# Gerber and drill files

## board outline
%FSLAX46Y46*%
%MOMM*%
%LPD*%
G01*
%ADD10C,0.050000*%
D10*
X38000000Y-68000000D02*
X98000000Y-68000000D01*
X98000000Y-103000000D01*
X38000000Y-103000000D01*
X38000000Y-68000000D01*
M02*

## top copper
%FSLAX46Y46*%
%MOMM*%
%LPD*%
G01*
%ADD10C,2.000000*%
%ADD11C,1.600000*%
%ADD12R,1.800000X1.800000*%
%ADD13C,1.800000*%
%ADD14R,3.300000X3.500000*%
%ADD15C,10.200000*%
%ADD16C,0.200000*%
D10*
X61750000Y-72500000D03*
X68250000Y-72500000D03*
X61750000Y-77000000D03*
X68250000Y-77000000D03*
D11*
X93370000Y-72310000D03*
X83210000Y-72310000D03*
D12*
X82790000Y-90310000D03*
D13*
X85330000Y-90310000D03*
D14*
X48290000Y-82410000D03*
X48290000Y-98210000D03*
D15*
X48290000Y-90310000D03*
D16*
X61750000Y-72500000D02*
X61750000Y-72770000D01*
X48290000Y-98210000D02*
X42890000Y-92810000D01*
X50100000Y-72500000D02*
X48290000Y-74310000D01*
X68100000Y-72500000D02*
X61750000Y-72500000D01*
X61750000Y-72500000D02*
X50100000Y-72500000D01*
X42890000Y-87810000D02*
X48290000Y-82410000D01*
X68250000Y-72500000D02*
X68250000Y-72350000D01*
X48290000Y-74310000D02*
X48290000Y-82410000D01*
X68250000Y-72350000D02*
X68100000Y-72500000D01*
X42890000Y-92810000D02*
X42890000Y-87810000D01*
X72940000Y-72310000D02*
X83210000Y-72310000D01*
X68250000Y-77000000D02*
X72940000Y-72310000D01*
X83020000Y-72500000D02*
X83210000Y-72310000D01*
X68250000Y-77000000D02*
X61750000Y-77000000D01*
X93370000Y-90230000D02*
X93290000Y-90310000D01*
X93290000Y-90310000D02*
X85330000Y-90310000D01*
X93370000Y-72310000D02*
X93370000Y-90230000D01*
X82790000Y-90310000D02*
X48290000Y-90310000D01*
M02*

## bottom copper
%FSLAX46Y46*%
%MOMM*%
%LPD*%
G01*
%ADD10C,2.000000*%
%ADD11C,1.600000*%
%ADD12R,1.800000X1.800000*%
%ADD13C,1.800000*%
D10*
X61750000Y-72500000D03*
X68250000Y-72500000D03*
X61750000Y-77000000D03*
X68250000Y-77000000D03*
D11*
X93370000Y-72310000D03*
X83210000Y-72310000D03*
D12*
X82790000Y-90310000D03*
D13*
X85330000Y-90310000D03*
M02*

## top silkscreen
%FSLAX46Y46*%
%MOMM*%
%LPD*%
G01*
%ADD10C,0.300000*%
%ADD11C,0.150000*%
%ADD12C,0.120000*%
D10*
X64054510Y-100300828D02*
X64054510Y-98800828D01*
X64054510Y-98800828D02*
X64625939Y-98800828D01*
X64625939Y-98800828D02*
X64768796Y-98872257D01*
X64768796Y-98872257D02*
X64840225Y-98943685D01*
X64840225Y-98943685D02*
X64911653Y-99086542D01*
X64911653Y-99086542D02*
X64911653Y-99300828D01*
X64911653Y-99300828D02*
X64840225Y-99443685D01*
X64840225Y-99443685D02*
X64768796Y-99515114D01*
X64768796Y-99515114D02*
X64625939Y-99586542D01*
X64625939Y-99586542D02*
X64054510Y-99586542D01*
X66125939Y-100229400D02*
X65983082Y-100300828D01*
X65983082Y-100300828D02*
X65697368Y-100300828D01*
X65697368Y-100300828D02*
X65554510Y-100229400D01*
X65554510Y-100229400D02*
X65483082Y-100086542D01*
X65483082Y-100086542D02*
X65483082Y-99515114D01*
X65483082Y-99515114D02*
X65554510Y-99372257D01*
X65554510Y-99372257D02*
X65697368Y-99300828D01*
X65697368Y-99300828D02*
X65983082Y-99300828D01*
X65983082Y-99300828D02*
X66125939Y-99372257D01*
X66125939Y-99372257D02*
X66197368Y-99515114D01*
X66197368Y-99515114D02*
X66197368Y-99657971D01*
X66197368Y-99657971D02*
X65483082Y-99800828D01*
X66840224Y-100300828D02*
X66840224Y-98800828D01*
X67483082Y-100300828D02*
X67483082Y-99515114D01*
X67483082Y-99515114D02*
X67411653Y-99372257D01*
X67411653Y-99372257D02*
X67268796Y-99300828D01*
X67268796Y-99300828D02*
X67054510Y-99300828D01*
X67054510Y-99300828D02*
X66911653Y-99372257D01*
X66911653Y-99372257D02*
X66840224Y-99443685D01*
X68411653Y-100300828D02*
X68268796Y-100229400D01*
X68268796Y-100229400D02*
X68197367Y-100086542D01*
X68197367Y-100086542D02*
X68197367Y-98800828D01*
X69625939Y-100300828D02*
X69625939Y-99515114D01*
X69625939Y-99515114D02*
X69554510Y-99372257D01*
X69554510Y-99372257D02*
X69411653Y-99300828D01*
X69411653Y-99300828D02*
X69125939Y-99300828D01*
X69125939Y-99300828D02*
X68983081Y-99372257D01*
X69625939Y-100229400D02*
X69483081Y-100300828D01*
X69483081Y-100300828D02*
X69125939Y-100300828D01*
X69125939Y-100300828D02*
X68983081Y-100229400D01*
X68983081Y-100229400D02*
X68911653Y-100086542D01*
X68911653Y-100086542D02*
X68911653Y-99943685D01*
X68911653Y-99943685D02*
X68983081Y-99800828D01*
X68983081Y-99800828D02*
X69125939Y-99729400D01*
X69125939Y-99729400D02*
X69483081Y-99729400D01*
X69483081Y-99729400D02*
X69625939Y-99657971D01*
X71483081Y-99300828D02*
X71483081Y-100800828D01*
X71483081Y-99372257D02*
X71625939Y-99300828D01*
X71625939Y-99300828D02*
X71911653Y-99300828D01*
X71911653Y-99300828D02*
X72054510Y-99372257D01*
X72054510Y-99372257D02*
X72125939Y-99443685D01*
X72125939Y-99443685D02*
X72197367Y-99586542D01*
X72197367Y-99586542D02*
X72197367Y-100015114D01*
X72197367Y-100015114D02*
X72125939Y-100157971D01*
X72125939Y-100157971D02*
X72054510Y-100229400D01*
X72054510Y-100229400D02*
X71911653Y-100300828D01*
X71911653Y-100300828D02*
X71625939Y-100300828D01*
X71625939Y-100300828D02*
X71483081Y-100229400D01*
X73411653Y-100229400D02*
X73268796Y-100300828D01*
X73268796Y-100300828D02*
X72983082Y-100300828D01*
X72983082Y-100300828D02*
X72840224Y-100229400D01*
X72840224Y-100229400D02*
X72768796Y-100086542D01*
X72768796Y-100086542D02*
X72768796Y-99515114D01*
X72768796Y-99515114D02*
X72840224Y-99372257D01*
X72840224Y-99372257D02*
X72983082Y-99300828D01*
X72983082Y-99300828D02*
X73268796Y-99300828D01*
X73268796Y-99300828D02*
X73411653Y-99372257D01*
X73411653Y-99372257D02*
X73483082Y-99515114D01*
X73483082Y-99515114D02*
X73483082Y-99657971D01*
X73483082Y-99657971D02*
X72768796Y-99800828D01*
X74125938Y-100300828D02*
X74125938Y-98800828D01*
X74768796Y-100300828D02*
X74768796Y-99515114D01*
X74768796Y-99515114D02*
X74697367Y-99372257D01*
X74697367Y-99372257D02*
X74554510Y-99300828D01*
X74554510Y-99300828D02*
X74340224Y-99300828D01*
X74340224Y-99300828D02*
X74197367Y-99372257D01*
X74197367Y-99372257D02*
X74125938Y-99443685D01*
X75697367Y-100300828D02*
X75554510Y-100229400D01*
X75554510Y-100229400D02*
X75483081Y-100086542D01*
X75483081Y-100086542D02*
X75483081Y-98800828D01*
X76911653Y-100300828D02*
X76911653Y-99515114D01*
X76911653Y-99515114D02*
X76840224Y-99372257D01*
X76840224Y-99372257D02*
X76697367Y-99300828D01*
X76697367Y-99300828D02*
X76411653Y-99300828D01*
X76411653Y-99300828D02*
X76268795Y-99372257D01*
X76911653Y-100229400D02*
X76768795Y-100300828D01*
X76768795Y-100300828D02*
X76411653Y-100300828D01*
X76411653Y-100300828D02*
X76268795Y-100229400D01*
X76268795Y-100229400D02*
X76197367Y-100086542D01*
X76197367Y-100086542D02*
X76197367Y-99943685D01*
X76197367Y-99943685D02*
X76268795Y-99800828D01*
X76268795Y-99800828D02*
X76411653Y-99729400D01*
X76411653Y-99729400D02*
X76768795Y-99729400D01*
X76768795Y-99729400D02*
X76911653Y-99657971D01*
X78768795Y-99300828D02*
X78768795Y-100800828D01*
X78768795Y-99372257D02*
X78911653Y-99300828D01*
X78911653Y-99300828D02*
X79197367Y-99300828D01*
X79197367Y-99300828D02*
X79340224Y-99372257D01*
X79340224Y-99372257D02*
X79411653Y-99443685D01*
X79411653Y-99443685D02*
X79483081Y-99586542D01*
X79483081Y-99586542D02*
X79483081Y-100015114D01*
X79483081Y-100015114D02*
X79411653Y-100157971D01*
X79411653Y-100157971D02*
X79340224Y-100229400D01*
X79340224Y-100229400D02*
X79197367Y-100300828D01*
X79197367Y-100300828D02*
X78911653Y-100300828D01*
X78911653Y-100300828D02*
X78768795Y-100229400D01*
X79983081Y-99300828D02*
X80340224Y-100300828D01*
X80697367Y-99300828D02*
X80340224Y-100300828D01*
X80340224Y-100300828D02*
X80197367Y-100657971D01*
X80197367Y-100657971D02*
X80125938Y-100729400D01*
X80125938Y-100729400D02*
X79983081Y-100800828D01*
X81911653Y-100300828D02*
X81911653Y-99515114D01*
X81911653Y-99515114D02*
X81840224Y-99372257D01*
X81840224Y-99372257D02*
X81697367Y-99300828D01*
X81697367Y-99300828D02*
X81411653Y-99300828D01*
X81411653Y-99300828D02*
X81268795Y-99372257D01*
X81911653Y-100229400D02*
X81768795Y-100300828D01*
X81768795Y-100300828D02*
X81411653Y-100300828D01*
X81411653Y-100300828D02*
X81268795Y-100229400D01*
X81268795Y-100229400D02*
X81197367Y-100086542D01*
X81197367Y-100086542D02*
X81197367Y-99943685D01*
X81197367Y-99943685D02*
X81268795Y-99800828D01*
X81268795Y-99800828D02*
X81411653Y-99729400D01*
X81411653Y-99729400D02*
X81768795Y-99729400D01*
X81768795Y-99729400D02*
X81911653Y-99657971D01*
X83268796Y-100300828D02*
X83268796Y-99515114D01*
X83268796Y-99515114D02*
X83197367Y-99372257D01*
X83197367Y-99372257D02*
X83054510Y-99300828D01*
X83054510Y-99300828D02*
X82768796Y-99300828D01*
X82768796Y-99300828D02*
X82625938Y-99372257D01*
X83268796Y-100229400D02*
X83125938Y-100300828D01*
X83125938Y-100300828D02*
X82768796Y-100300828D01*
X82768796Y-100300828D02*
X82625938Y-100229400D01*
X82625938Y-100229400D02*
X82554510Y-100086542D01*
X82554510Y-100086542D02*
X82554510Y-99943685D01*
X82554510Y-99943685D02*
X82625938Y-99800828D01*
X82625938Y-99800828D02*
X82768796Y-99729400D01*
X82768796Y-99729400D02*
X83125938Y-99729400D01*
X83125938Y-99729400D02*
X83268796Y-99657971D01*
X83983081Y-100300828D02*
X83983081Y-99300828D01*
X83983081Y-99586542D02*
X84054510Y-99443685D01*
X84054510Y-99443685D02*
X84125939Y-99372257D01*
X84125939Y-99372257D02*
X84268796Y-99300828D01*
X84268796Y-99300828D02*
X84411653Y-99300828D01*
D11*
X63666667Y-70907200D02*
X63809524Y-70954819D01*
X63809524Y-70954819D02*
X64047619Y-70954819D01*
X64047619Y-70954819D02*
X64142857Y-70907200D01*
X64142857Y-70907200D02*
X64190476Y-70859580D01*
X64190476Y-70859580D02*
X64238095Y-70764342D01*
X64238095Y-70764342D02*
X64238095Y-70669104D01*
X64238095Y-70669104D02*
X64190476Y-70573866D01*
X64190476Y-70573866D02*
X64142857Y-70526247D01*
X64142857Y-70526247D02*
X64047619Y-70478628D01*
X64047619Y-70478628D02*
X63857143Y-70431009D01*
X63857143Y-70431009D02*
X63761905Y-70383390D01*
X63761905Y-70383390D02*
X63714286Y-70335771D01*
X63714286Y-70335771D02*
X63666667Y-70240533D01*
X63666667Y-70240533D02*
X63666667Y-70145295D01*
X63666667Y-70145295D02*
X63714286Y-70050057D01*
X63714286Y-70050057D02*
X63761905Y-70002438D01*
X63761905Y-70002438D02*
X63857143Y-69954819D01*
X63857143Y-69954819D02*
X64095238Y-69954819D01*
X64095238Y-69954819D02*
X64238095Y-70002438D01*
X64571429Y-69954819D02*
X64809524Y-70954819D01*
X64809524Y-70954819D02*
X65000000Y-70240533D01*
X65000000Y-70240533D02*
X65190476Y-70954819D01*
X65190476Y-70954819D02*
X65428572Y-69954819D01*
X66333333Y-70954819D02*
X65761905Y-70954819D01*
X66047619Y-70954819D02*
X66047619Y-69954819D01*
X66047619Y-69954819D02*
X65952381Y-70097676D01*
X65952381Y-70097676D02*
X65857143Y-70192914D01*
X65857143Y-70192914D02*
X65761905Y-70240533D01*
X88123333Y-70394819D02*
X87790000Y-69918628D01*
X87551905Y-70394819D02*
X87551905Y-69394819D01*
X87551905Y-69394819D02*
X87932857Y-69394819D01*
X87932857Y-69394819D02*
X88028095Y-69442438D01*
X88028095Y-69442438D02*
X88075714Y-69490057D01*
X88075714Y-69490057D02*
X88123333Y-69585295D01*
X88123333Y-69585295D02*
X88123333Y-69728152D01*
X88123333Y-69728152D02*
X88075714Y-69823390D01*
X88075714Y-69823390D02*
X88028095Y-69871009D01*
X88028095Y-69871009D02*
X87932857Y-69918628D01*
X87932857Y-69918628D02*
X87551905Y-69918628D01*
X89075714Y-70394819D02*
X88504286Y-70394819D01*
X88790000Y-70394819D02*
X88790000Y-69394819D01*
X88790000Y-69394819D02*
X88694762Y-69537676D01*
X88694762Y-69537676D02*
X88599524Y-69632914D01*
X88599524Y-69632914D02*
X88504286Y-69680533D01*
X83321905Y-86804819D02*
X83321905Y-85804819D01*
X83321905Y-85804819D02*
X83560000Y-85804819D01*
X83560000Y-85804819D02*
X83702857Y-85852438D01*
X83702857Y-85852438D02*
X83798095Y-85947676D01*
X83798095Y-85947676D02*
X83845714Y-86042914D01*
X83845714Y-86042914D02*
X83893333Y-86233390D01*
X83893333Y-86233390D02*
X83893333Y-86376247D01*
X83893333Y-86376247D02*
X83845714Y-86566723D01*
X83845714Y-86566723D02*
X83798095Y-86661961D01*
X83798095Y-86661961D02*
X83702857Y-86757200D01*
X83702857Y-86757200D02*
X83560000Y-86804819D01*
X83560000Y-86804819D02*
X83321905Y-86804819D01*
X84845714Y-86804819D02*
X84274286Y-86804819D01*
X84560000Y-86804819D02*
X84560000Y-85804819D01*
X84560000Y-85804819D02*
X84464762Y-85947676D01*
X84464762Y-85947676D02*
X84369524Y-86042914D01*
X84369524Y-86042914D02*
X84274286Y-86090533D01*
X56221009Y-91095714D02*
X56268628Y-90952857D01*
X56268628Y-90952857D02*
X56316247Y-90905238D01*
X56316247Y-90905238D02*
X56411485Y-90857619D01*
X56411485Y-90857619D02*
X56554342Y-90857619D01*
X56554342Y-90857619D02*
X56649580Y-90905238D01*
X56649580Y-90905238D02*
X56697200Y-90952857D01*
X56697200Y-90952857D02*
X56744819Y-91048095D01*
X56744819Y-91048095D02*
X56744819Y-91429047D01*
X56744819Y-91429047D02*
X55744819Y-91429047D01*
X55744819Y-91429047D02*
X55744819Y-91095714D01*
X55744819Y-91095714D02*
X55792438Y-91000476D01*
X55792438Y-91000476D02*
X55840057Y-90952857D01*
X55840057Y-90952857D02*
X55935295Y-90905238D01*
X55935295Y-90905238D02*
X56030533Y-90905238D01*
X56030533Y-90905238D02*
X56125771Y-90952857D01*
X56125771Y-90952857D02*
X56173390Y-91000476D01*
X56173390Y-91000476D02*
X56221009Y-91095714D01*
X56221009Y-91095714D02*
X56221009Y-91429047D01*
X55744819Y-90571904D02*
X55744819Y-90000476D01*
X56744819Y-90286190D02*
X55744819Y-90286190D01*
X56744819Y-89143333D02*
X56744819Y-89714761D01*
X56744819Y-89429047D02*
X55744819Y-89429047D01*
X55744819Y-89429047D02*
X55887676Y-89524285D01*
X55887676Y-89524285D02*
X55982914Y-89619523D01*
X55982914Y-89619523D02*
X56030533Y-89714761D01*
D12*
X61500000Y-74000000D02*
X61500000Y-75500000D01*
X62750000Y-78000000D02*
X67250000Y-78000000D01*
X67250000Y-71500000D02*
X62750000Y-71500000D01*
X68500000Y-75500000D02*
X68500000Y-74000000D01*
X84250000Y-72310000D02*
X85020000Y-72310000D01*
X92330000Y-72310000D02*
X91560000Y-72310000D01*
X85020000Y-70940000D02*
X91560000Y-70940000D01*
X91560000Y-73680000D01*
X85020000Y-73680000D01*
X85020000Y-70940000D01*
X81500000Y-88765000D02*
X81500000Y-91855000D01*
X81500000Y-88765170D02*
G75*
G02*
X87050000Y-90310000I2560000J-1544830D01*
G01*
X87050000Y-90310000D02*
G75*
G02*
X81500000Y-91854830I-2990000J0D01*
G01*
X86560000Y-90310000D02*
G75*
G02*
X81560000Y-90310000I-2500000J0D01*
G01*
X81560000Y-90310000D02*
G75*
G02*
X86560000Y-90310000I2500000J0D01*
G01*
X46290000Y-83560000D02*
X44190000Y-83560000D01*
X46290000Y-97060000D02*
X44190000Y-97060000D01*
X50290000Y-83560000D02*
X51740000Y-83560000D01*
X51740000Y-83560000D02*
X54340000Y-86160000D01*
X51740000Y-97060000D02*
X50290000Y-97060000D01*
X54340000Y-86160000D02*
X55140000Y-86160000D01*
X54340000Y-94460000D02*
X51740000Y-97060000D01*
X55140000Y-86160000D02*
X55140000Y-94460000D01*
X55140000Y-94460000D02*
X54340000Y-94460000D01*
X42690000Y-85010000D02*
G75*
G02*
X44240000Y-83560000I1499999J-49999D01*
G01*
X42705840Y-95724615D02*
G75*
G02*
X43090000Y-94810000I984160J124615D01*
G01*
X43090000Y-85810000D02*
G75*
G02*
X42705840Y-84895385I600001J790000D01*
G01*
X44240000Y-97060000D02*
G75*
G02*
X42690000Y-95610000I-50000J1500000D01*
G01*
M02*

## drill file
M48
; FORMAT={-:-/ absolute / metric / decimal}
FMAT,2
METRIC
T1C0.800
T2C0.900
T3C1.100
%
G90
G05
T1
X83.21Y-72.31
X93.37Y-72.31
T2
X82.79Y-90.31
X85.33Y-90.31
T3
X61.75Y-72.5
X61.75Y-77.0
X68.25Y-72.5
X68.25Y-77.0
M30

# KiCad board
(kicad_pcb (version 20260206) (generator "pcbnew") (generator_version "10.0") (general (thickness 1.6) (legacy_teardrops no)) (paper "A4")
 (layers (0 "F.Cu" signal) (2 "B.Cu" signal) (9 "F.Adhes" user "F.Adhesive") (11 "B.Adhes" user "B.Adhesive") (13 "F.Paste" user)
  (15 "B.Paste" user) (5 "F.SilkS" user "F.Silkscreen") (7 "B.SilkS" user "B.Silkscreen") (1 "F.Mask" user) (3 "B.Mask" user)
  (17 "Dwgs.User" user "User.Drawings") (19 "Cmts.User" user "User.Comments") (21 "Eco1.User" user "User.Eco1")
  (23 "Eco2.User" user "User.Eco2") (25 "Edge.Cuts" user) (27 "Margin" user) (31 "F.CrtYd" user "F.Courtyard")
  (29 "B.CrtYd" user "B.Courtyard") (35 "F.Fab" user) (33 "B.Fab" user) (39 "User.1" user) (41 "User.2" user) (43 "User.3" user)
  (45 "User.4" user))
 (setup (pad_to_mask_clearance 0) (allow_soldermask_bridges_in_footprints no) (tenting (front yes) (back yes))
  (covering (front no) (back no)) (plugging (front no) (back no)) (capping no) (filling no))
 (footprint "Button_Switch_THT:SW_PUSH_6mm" (layer "F.Cu") (at 61.75 72.5)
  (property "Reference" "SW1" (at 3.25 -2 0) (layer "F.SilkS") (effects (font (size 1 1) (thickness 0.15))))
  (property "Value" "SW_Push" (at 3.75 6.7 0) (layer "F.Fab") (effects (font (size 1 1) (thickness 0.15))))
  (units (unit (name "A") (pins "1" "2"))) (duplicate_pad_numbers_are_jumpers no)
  (fp_line (start -0.25 1.5) (end -0.25 3) (stroke (width 0.12) (type solid)) (layer "F.SilkS"))
  (fp_line (start 1 5.5) (end 5.5 5.5) (stroke (width 0.12) (type solid)) (layer "F.SilkS"))
  (fp_line (start 5.5 -1) (end 1 -1) (stroke (width 0.12) (type solid)) (layer "F.SilkS"))
  (fp_line (start 6.75 3) (end 6.75 1.5) (stroke (width 0.12) (type solid)) (layer "F.SilkS"))
  (pad "1" thru_hole circle (at 0 0 90) (size 2 2) (drill 1.1) (layers "*.Cu" "*.Mask") (remove_unused_layers no) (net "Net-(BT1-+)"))
  (pad "1" thru_hole circle (at 6.5 0 90) (size 2 2) (drill 1.1) (layers "*.Cu" "*.Mask") (remove_unused_layers no) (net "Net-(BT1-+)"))
  (pad "2" thru_hole circle (at 0 4.5 90) (size 2 2) (drill 1.1) (layers "*.Cu" "*.Mask") (remove_unused_layers no) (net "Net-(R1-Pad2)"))
  (pad "2" thru_hole circle (at 6.5 4.5 90) (size 2 2) (drill 1.1) (layers "*.Cu" "*.Mask") (remove_unused_layers no) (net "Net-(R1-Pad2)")))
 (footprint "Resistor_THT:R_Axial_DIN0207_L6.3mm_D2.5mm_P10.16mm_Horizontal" (layer "F.Cu") (at 93.37 72.31 180)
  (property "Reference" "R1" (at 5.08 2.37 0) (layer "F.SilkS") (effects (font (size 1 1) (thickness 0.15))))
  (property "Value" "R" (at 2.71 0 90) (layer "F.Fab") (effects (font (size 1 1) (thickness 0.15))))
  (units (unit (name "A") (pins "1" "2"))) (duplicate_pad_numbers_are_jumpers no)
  (fp_line (start 9.12 0) (end 8.35 0) (stroke (width 0.12) (type solid)) (layer "F.SilkS"))
  (fp_line (start 1.04 0) (end 1.81 0) (stroke (width 0.12) (type solid)) (layer "F.SilkS"))
  (fp_rect (start 1.81 -1.37) (end 8.35 1.37) (stroke (width 0.12) (type solid)) (fill no) (layer "F.SilkS"))
  (pad "1" thru_hole circle (at 0 0 180) (size 1.6 1.6) (drill 0.8) (layers "*.Cu" "*.Mask") (remove_unused_layers no) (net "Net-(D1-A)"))
  (pad "2" thru_hole circle (at 10.16 0 180) (size 1.6 1.6) (drill 0.8) (layers "*.Cu" "*.Mask") (remove_unused_layers no)
   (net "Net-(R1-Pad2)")))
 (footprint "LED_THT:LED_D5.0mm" (layer "F.Cu") (at 82.79 90.31)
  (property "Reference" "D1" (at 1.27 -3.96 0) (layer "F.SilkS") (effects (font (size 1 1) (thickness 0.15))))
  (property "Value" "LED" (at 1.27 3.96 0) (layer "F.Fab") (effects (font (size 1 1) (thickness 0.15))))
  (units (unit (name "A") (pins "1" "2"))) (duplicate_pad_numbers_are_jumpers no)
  (fp_line (start -1.29 -1.545) (end -1.29 1.545) (stroke (width 0.12) (type solid)) (layer "F.SilkS"))
  (fp_arc (start -1.29 -1.54483) (mid 2.071779 -2.880495) (end 4.26 0) (stroke (width 0.12) (type solid)) (layer "F.SilkS"))
  (fp_arc (start 4.26 0) (mid 2.071779 2.880495) (end -1.29 1.54483) (stroke (width 0.12) (type solid)) (layer "F.SilkS"))
  (fp_circle (center 1.27 0) (end 3.77 0) (stroke (width 0.12) (type solid)) (fill no) (layer "F.SilkS"))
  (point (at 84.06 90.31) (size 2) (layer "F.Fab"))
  (pad "1" thru_hole rect (at 0 0) (size 1.8 1.8) (drill 0.9) (layers "*.Cu" "*.Mask") (remove_unused_layers no) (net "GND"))
  (pad "2" thru_hole circle (at 2.54 0) (size 1.8 1.8) (drill 0.9) (layers "*.Cu" "*.Mask") (remove_unused_layers no) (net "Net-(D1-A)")))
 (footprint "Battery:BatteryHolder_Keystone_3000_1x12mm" (layer "F.Cu") (at 48.29 90.31 -90)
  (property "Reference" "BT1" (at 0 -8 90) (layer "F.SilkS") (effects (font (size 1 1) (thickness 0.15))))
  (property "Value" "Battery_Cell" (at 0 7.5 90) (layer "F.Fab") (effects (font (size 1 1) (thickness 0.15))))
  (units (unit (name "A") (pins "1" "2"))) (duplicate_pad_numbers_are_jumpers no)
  (fp_line (start -6.75 2) (end -6.75 4.1) (stroke (width 0.12) (type solid)) (layer "F.SilkS"))
  (fp_line (start 6.75 2) (end 6.75 4.1) (stroke (width 0.12) (type solid)) (layer "F.SilkS"))
  (fp_line (start -6.75 -2) (end -6.75 -3.45) (stroke (width 0.12) (type solid)) (layer "F.SilkS"))
  (fp_line (start -6.75 -3.45) (end -4.15 -6.05) (stroke (width 0.12) (type solid)) (layer "F.SilkS"))
  (fp_line (start 6.75 -3.45) (end 6.75 -2) (stroke (width 0.12) (type solid)) (layer "F.SilkS"))
  (fp_line (start -4.15 -6.05) (end -4.15 -6.85) (stroke (width 0.12) (type solid)) (layer "F.SilkS"))
  (fp_line (start 4.15 -6.05) (end 6.75 -3.45) (stroke (width 0.12) (type solid)) (layer "F.SilkS"))
  (fp_line (start -4.15 -6.85) (end 4.15 -6.85) (stroke (width 0.12) (type solid)) (layer "F.SilkS"))
  (fp_line (start 4.15 -6.85) (end 4.15 -6.05) (stroke (width 0.12) (type solid)) (layer "F.SilkS"))
  (fp_arc (start -5.3 5.6) (mid -6.346016 5.125305) (end -6.75 4.05) (stroke (width 0.12) (type solid)) (layer "F.SilkS"))
  (fp_arc (start 5.414615 5.58416) (mid 4.90584 5.514615) (end 4.5 5.2) (stroke (width 0.12) (type solid)) (layer "F.SilkS"))
  (fp_arc (start -4.5 5.2) (mid -4.90584 5.514615) (end -5.414615 5.58416) (stroke (width 0.12) (type solid)) (layer "F.SilkS"))
  (fp_arc (start 6.75 4.05) (mid 6.346016 5.125305) (end 5.3 5.6) (stroke (width 0.12) (type solid)) (layer "F.SilkS"))
  (pad "1" smd rect (at -7.9 0 270) (size 3.5 3.3) (layers "F.Cu" "F.Mask" "F.Paste") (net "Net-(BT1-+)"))
  (pad "1" smd rect (at 7.9 0 270) (size 3.5 3.3) (layers "F.Cu" "F.Mask" "F.Paste") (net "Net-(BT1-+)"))
  (pad "2" smd circle (at 0 0 270) (size 10.2 10.2) (layers "F.Cu" "F.Mask") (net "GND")))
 (gr_rect (start 38 68) (end 98 103) (stroke (width 0.05) (type default)) (fill no) (layer "Edge.Cuts"))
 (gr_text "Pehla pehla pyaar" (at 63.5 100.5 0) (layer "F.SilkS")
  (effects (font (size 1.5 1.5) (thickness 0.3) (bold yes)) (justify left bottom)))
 (segment (start 61.75 72.5) (end 61.75 72.77) (width 0.2) (layer "F.Cu") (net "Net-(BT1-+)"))
 (segment (start 48.29 98.21) (end 42.89 92.81) (width 0.2) (layer "F.Cu") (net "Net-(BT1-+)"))
 (segment (start 50.1 72.5) (end 48.29 74.31) (width 0.2) (layer "F.Cu") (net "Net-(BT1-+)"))
 (segment (start 68.1 72.5) (end 61.75 72.5) (width 0.2) (layer "F.Cu") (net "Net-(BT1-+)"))
 (segment (start 61.75 72.5) (end 50.1 72.5) (width 0.2) (layer "F.Cu") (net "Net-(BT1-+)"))
 (segment (start 42.89 87.81) (end 48.29 82.41) (width 0.2) (layer "F.Cu") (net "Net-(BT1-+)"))
 (segment (start 68.25 72.5) (end 68.25 72.35) (width 0.2) (layer "F.Cu") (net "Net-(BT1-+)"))
 (segment (start 48.29 74.31) (end 48.29 82.41) (width 0.2) (layer "F.Cu") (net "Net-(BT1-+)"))
 (segment (start 68.25 72.35) (end 68.1 72.5) (width 0.2) (layer "F.Cu") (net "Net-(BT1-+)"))
 (segment (start 42.89 92.81) (end 42.89 87.81) (width 0.2) (layer "F.Cu") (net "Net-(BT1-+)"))
 (segment (start 72.94 72.31) (end 83.21 72.31) (width 0.2) (layer "F.Cu") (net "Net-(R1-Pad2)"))
 (segment (start 68.25 77) (end 72.94 72.31) (width 0.2) (layer "F.Cu") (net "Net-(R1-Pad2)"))
 (segment (start 83.02 72.5) (end 83.21 72.31) (width 0.2) (layer "F.Cu") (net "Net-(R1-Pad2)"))
 (segment (start 68.25 77) (end 61.75 77) (width 0.2) (layer "F.Cu") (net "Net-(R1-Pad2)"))
 (segment (start 93.37 90.23) (end 93.29 90.31) (width 0.2) (layer "F.Cu") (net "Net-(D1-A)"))
 (segment (start 93.29 90.31) (end 85.33 90.31) (width 0.2) (layer "F.Cu") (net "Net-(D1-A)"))
 (segment (start 93.37 72.31) (end 93.37 90.23) (width 0.2) (layer "F.Cu") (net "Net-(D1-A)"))
 (segment (start 82.79 90.31) (end 48.29 90.31) (width 0.2) (layer "F.Cu") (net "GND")))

